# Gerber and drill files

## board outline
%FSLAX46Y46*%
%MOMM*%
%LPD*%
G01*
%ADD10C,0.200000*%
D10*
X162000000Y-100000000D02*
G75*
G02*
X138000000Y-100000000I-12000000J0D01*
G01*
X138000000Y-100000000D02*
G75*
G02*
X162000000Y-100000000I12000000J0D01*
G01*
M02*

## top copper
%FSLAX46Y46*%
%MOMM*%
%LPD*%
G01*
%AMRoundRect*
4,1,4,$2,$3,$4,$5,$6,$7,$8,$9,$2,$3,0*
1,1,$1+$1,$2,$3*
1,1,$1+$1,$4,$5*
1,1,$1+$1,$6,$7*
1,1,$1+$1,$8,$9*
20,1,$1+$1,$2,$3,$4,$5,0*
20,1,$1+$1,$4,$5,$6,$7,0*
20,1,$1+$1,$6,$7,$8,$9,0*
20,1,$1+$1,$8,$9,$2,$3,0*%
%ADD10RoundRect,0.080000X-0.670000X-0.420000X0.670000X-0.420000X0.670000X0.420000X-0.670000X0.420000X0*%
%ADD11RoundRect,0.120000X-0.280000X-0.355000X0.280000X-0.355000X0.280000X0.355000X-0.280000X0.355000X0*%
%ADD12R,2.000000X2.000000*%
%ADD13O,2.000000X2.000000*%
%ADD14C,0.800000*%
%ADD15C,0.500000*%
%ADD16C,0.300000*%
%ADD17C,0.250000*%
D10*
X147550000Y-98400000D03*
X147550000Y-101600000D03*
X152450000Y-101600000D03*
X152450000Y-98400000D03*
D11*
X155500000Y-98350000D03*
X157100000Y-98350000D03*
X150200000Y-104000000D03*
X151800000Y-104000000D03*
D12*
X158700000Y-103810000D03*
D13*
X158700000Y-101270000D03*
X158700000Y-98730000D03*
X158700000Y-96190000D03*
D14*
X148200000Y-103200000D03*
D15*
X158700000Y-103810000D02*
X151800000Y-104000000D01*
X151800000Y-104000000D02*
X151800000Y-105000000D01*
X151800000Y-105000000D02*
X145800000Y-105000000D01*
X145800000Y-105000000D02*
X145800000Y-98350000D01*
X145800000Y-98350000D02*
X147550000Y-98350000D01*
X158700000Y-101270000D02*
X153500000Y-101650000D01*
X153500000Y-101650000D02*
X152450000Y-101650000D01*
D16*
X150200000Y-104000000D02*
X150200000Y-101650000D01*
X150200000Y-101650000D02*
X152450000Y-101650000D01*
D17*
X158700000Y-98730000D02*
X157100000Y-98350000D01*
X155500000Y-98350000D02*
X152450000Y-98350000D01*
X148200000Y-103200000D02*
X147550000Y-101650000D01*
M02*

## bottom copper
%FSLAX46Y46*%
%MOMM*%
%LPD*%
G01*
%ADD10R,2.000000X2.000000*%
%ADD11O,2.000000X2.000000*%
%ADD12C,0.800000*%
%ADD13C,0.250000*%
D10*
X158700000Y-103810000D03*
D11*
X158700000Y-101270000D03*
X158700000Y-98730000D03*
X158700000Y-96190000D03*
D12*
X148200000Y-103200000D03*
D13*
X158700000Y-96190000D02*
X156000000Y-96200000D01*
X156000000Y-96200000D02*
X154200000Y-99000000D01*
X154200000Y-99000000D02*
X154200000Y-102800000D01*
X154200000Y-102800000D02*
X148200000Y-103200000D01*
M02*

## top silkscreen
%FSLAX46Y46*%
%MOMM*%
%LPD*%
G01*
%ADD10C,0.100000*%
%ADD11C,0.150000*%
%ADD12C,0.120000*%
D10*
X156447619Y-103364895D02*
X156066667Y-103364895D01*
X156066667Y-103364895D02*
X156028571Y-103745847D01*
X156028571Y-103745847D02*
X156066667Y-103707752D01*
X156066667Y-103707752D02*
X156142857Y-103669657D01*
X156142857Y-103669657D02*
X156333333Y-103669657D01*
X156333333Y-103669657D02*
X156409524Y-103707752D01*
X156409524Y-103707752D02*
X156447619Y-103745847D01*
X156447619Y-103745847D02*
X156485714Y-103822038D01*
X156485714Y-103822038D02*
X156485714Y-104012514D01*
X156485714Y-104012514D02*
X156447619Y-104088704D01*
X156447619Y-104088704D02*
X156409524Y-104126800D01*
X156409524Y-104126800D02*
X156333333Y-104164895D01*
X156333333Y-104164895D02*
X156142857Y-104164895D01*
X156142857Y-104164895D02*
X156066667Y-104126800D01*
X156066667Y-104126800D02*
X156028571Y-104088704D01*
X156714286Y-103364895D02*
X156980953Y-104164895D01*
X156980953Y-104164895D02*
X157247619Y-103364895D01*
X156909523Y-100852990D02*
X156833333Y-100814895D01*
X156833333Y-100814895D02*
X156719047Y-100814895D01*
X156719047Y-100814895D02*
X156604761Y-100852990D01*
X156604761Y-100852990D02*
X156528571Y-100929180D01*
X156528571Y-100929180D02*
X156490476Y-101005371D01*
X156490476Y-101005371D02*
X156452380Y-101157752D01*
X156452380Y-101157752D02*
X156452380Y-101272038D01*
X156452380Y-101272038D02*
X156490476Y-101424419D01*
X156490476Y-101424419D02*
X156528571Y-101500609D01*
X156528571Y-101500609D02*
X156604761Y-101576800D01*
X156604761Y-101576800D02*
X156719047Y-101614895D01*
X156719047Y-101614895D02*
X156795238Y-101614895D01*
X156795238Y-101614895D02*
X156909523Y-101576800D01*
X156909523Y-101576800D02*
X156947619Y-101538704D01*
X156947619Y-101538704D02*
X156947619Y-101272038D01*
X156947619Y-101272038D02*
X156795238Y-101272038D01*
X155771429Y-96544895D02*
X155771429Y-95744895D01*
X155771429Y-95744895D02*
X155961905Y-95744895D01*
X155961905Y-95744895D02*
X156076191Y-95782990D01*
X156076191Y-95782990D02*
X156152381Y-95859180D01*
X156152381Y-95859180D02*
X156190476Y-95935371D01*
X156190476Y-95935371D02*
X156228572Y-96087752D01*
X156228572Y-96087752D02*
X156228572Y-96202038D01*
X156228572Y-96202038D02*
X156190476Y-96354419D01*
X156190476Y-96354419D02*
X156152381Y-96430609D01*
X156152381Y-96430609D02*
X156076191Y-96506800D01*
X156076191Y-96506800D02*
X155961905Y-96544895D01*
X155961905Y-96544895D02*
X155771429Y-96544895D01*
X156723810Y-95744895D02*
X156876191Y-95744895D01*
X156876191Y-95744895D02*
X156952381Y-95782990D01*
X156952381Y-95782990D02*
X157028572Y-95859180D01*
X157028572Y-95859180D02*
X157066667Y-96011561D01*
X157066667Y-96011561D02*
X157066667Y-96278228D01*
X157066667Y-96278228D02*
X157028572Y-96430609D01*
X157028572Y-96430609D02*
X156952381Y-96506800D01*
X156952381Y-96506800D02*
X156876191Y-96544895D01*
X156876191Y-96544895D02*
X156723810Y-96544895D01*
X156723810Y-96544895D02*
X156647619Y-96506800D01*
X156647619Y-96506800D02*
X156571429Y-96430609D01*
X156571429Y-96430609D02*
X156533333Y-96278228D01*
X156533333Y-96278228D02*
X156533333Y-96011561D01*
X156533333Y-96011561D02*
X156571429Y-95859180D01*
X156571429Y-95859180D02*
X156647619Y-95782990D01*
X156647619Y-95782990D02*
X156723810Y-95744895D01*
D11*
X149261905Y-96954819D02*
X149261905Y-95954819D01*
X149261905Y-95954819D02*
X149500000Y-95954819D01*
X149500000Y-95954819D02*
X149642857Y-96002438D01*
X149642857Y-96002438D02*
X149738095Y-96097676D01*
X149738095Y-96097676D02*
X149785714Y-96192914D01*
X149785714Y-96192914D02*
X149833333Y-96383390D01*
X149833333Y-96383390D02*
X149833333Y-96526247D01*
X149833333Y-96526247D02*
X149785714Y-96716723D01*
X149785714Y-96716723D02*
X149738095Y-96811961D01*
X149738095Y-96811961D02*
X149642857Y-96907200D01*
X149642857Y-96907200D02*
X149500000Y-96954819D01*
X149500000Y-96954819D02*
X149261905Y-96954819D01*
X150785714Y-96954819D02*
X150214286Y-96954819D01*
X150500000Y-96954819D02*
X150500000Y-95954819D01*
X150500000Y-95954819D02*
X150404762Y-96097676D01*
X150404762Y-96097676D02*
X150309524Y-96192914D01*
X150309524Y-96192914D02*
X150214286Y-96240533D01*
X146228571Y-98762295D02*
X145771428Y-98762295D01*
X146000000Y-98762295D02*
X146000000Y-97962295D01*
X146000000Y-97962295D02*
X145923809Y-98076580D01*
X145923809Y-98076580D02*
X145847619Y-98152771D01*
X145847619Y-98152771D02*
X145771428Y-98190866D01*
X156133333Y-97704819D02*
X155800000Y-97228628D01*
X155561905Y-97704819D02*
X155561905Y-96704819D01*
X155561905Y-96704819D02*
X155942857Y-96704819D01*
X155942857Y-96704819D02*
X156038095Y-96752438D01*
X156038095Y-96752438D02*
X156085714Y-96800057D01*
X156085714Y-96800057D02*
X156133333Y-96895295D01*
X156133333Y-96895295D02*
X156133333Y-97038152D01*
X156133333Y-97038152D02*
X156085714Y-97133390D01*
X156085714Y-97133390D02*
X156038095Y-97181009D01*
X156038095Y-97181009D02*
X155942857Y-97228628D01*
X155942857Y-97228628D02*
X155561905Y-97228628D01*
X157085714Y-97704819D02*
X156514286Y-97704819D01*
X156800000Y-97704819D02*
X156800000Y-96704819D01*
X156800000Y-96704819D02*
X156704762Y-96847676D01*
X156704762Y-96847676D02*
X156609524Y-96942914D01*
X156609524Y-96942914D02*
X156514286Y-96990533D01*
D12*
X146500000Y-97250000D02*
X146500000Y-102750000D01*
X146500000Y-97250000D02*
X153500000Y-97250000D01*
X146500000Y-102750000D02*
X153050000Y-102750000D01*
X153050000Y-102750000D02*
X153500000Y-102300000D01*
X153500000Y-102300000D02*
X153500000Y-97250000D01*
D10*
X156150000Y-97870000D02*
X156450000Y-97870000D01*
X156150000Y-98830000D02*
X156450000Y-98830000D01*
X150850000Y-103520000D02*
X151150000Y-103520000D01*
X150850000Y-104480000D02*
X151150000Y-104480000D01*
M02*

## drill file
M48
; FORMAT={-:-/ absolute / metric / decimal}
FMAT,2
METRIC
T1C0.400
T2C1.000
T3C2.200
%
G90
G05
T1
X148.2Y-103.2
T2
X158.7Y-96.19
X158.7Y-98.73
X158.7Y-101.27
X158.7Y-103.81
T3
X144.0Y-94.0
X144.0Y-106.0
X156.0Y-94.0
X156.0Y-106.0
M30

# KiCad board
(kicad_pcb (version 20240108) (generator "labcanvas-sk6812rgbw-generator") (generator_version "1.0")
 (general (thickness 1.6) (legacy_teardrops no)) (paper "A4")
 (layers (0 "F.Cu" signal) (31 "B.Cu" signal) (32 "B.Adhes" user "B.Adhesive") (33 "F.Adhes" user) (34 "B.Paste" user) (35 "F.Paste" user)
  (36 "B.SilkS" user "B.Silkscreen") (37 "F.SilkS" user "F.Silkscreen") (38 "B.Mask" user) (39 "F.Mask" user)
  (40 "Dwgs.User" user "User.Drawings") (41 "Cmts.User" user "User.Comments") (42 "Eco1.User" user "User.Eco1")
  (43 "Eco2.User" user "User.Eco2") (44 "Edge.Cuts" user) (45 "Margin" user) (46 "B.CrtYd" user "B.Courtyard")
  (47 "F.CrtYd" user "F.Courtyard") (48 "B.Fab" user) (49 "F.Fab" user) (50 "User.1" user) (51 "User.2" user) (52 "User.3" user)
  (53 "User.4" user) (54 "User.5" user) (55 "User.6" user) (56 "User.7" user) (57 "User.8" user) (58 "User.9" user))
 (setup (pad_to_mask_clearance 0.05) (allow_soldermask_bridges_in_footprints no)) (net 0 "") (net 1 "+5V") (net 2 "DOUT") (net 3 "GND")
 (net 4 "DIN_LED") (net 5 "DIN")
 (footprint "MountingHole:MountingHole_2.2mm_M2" (layer "F.Cu") (at 144 94)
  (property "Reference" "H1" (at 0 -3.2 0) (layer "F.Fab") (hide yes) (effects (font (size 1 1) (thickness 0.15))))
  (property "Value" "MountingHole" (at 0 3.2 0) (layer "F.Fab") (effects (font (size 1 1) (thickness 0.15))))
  (pad "" np_thru_hole circle (at 0 0) (size 2.2 2.2) (drill 2.2) (layers "*.Cu" "*.Mask")))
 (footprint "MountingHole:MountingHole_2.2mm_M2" (layer "F.Cu") (at 156 94)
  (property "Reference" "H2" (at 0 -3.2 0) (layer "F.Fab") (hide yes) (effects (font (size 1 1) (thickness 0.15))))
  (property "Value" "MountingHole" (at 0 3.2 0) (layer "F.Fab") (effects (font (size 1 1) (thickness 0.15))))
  (pad "" np_thru_hole circle (at 0 0) (size 2.2 2.2) (drill 2.2) (layers "*.Cu" "*.Mask")))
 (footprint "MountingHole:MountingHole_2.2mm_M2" (layer "F.Cu") (at 156 106)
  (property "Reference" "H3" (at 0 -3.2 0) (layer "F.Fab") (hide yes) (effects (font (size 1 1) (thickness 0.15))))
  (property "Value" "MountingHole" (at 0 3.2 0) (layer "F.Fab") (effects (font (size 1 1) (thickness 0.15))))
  (pad "" np_thru_hole circle (at 0 0) (size 2.2 2.2) (drill 2.2) (layers "*.Cu" "*.Mask")))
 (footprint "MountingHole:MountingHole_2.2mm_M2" (layer "F.Cu") (at 144 106)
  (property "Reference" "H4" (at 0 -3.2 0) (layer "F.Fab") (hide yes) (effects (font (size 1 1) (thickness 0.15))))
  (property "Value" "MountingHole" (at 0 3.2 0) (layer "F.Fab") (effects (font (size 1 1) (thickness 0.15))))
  (pad "" np_thru_hole circle (at 0 0) (size 2.2 2.2) (drill 2.2) (layers "*.Cu" "*.Mask")))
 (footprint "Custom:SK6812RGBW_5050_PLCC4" (layer "F.Cu") (at 150 100)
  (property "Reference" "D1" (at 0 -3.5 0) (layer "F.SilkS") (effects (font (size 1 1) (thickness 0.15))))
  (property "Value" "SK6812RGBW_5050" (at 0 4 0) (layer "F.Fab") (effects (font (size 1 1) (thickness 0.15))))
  (fp_line (start -3.5 -2.75) (end -3.5 2.75) (stroke (width 0.12) (type solid)) (layer "F.SilkS"))
  (fp_line (start -3.5 -2.75) (end 3.5 -2.75) (stroke (width 0.12) (type solid)) (layer "F.SilkS"))
  (fp_line (start -3.5 2.75) (end 3.05 2.75) (stroke (width 0.12) (type solid)) (layer "F.SilkS"))
  (fp_line (start 3.05 2.75) (end 3.5 2.3) (stroke (width 0.12) (type solid)) (layer "F.SilkS"))
  (fp_line (start 3.5 2.3) (end 3.5 -2.75) (stroke (width 0.12) (type solid)) (layer "F.SilkS"))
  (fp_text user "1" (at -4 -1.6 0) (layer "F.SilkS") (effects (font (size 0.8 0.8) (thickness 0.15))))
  (pad "1" smd roundrect (at -2.45 -1.6) (size 1.5 1.0) (layers "F.Cu" "F.Mask" "F.Paste") (roundrect_rratio 0.08) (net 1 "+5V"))
  (pad "2" smd roundrect (at -2.45 1.6) (size 1.5 1.0) (layers "F.Cu" "F.Mask" "F.Paste") (roundrect_rratio 0.08) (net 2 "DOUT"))
  (pad "3" smd roundrect (at 2.45 1.6) (size 1.5 1.0) (layers "F.Cu" "F.Mask" "F.Paste") (roundrect_rratio 0.08) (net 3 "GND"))
  (pad "4" smd roundrect (at 2.45 -1.6) (size 1.5 1.0) (layers "F.Cu" "F.Mask" "F.Paste") (roundrect_rratio 0.08) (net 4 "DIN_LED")))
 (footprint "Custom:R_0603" (layer "F.Cu") (at 156.3 98.35)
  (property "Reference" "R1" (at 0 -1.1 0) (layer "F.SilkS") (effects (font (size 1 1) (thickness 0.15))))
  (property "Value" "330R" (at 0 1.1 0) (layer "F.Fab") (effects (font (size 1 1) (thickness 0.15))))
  (fp_line (start -0.15 -0.48) (end 0.15 -0.48) (stroke (width 0.10) (type solid)) (layer "F.SilkS"))
  (fp_line (start -0.15 0.48) (end 0.15 0.48) (stroke (width 0.10) (type solid)) (layer "F.SilkS"))
  (pad "1" smd roundrect (at -0.8 0) (size 0.8 0.95) (layers "F.Cu" "F.Mask" "F.Paste") (roundrect_rratio 0.15) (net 4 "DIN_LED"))
  (pad "2" smd roundrect (at 0.8 0) (size 0.8 0.95) (layers "F.Cu" "F.Mask" "F.Paste") (roundrect_rratio 0.15) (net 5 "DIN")))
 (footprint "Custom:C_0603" (layer "F.Cu") (at 151 104)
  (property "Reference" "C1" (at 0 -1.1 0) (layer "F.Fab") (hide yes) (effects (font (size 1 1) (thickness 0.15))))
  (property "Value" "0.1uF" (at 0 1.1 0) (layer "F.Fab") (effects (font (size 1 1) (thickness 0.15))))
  (fp_line (start -0.15 -0.48) (end 0.15 -0.48) (stroke (width 0.10) (type solid)) (layer "F.SilkS"))
  (fp_line (start -0.15 0.48) (end 0.15 0.48) (stroke (width 0.10) (type solid)) (layer "F.SilkS"))
  (pad "1" smd roundrect (at -0.8 0) (size 0.8 0.95) (layers "F.Cu" "F.Mask" "F.Paste") (roundrect_rratio 0.15) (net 3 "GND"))
  (pad "2" smd roundrect (at 0.8 0) (size 0.8 0.95) (layers "F.Cu" "F.Mask" "F.Paste") (roundrect_rratio 0.15) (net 1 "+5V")))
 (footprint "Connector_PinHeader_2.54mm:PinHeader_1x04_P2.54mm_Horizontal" (layer "B.Cu") (at 158.7 103.81)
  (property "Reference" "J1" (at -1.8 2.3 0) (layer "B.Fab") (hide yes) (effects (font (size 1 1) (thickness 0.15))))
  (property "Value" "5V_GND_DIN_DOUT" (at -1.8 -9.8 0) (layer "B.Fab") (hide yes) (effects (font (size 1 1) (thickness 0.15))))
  (pad "1" thru_hole rect (at 0 0) (size 2.0 2.0) (drill 1.0) (layers "*.Cu" "*.Mask") (remove_unused_layers no) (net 1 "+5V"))
  (pad "2" thru_hole oval (at 0 -2.54) (size 2.0 2.0) (drill 1.0) (layers "*.Cu" "*.Mask") (remove_unused_layers no) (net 3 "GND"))
  (pad "3" thru_hole oval (at 0 -5.08) (size 2.0 2.0) (drill 1.0) (layers "*.Cu" "*.Mask") (remove_unused_layers no) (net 5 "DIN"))
  (pad "4" thru_hole oval (at 0 -7.62) (size 2.0 2.0) (drill 1.0) (layers "*.Cu" "*.Mask") (remove_unused_layers no) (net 2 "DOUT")))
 (gr_circle (center 150 100) (end 162 100) (stroke (width 0.2) (type default)) (fill none) (layer "Edge.Cuts"))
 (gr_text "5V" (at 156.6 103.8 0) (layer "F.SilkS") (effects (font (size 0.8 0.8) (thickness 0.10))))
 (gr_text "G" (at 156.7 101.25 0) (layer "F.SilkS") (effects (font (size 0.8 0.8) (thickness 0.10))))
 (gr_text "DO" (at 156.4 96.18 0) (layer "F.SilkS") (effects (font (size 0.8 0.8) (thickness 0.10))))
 (segment (start 158.7 103.81) (end 151.8 104) (width 0.5) (layer "F.Cu") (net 1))
 (segment (start 151.8 104) (end 151.8 105) (width 0.5) (layer "F.Cu") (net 1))
 (segment (start 151.8 105) (end 145.8 105) (width 0.5) (layer "F.Cu") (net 1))
 (segment (start 145.8 105) (end 145.8 98.35) (width 0.5) (layer "F.Cu") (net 1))
 (segment (start 145.8 98.35) (end 147.55 98.35) (width 0.5) (layer "F.Cu") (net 1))
 (segment (start 158.7 101.27) (end 153.5 101.65) (width 0.5) (layer "F.Cu") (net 3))
 (segment (start 153.5 101.65) (end 152.45 101.65) (width 0.5) (layer "F.Cu") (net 3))
 (segment (start 150.2 104) (end 150.2 101.65) (width 0.3) (layer "F.Cu") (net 3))
 (segment (start 150.2 101.65) (end 152.45 101.65) (width 0.3) (layer "F.Cu") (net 3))
 (segment (start 158.7 98.73) (end 157.1 98.35) (width 0.25) (layer "F.Cu") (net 5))
 (segment (start 155.5 98.35) (end 152.45 98.35) (width 0.25) (layer "F.Cu") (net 4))
 (segment (start 158.7 96.19) (end 156 96.2) (width 0.25) (layer "B.Cu") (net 2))
 (segment (start 156 96.2) (end 154.2 99.0) (width 0.25) (layer "B.Cu") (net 2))
 (segment (start 154.2 99.0) (end 154.2 102.8) (width 0.25) (layer "B.Cu") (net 2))
 (segment (start 154.2 102.8) (end 148.2 103.2) (width 0.25) (layer "B.Cu") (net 2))
 (via (at 148.2 103.2) (size 0.8) (drill 0.4) (layers "F.Cu" "B.Cu") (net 2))
 (segment (start 148.2 103.2) (end 147.55 101.65) (width 0.25) (layer "F.Cu") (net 2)))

